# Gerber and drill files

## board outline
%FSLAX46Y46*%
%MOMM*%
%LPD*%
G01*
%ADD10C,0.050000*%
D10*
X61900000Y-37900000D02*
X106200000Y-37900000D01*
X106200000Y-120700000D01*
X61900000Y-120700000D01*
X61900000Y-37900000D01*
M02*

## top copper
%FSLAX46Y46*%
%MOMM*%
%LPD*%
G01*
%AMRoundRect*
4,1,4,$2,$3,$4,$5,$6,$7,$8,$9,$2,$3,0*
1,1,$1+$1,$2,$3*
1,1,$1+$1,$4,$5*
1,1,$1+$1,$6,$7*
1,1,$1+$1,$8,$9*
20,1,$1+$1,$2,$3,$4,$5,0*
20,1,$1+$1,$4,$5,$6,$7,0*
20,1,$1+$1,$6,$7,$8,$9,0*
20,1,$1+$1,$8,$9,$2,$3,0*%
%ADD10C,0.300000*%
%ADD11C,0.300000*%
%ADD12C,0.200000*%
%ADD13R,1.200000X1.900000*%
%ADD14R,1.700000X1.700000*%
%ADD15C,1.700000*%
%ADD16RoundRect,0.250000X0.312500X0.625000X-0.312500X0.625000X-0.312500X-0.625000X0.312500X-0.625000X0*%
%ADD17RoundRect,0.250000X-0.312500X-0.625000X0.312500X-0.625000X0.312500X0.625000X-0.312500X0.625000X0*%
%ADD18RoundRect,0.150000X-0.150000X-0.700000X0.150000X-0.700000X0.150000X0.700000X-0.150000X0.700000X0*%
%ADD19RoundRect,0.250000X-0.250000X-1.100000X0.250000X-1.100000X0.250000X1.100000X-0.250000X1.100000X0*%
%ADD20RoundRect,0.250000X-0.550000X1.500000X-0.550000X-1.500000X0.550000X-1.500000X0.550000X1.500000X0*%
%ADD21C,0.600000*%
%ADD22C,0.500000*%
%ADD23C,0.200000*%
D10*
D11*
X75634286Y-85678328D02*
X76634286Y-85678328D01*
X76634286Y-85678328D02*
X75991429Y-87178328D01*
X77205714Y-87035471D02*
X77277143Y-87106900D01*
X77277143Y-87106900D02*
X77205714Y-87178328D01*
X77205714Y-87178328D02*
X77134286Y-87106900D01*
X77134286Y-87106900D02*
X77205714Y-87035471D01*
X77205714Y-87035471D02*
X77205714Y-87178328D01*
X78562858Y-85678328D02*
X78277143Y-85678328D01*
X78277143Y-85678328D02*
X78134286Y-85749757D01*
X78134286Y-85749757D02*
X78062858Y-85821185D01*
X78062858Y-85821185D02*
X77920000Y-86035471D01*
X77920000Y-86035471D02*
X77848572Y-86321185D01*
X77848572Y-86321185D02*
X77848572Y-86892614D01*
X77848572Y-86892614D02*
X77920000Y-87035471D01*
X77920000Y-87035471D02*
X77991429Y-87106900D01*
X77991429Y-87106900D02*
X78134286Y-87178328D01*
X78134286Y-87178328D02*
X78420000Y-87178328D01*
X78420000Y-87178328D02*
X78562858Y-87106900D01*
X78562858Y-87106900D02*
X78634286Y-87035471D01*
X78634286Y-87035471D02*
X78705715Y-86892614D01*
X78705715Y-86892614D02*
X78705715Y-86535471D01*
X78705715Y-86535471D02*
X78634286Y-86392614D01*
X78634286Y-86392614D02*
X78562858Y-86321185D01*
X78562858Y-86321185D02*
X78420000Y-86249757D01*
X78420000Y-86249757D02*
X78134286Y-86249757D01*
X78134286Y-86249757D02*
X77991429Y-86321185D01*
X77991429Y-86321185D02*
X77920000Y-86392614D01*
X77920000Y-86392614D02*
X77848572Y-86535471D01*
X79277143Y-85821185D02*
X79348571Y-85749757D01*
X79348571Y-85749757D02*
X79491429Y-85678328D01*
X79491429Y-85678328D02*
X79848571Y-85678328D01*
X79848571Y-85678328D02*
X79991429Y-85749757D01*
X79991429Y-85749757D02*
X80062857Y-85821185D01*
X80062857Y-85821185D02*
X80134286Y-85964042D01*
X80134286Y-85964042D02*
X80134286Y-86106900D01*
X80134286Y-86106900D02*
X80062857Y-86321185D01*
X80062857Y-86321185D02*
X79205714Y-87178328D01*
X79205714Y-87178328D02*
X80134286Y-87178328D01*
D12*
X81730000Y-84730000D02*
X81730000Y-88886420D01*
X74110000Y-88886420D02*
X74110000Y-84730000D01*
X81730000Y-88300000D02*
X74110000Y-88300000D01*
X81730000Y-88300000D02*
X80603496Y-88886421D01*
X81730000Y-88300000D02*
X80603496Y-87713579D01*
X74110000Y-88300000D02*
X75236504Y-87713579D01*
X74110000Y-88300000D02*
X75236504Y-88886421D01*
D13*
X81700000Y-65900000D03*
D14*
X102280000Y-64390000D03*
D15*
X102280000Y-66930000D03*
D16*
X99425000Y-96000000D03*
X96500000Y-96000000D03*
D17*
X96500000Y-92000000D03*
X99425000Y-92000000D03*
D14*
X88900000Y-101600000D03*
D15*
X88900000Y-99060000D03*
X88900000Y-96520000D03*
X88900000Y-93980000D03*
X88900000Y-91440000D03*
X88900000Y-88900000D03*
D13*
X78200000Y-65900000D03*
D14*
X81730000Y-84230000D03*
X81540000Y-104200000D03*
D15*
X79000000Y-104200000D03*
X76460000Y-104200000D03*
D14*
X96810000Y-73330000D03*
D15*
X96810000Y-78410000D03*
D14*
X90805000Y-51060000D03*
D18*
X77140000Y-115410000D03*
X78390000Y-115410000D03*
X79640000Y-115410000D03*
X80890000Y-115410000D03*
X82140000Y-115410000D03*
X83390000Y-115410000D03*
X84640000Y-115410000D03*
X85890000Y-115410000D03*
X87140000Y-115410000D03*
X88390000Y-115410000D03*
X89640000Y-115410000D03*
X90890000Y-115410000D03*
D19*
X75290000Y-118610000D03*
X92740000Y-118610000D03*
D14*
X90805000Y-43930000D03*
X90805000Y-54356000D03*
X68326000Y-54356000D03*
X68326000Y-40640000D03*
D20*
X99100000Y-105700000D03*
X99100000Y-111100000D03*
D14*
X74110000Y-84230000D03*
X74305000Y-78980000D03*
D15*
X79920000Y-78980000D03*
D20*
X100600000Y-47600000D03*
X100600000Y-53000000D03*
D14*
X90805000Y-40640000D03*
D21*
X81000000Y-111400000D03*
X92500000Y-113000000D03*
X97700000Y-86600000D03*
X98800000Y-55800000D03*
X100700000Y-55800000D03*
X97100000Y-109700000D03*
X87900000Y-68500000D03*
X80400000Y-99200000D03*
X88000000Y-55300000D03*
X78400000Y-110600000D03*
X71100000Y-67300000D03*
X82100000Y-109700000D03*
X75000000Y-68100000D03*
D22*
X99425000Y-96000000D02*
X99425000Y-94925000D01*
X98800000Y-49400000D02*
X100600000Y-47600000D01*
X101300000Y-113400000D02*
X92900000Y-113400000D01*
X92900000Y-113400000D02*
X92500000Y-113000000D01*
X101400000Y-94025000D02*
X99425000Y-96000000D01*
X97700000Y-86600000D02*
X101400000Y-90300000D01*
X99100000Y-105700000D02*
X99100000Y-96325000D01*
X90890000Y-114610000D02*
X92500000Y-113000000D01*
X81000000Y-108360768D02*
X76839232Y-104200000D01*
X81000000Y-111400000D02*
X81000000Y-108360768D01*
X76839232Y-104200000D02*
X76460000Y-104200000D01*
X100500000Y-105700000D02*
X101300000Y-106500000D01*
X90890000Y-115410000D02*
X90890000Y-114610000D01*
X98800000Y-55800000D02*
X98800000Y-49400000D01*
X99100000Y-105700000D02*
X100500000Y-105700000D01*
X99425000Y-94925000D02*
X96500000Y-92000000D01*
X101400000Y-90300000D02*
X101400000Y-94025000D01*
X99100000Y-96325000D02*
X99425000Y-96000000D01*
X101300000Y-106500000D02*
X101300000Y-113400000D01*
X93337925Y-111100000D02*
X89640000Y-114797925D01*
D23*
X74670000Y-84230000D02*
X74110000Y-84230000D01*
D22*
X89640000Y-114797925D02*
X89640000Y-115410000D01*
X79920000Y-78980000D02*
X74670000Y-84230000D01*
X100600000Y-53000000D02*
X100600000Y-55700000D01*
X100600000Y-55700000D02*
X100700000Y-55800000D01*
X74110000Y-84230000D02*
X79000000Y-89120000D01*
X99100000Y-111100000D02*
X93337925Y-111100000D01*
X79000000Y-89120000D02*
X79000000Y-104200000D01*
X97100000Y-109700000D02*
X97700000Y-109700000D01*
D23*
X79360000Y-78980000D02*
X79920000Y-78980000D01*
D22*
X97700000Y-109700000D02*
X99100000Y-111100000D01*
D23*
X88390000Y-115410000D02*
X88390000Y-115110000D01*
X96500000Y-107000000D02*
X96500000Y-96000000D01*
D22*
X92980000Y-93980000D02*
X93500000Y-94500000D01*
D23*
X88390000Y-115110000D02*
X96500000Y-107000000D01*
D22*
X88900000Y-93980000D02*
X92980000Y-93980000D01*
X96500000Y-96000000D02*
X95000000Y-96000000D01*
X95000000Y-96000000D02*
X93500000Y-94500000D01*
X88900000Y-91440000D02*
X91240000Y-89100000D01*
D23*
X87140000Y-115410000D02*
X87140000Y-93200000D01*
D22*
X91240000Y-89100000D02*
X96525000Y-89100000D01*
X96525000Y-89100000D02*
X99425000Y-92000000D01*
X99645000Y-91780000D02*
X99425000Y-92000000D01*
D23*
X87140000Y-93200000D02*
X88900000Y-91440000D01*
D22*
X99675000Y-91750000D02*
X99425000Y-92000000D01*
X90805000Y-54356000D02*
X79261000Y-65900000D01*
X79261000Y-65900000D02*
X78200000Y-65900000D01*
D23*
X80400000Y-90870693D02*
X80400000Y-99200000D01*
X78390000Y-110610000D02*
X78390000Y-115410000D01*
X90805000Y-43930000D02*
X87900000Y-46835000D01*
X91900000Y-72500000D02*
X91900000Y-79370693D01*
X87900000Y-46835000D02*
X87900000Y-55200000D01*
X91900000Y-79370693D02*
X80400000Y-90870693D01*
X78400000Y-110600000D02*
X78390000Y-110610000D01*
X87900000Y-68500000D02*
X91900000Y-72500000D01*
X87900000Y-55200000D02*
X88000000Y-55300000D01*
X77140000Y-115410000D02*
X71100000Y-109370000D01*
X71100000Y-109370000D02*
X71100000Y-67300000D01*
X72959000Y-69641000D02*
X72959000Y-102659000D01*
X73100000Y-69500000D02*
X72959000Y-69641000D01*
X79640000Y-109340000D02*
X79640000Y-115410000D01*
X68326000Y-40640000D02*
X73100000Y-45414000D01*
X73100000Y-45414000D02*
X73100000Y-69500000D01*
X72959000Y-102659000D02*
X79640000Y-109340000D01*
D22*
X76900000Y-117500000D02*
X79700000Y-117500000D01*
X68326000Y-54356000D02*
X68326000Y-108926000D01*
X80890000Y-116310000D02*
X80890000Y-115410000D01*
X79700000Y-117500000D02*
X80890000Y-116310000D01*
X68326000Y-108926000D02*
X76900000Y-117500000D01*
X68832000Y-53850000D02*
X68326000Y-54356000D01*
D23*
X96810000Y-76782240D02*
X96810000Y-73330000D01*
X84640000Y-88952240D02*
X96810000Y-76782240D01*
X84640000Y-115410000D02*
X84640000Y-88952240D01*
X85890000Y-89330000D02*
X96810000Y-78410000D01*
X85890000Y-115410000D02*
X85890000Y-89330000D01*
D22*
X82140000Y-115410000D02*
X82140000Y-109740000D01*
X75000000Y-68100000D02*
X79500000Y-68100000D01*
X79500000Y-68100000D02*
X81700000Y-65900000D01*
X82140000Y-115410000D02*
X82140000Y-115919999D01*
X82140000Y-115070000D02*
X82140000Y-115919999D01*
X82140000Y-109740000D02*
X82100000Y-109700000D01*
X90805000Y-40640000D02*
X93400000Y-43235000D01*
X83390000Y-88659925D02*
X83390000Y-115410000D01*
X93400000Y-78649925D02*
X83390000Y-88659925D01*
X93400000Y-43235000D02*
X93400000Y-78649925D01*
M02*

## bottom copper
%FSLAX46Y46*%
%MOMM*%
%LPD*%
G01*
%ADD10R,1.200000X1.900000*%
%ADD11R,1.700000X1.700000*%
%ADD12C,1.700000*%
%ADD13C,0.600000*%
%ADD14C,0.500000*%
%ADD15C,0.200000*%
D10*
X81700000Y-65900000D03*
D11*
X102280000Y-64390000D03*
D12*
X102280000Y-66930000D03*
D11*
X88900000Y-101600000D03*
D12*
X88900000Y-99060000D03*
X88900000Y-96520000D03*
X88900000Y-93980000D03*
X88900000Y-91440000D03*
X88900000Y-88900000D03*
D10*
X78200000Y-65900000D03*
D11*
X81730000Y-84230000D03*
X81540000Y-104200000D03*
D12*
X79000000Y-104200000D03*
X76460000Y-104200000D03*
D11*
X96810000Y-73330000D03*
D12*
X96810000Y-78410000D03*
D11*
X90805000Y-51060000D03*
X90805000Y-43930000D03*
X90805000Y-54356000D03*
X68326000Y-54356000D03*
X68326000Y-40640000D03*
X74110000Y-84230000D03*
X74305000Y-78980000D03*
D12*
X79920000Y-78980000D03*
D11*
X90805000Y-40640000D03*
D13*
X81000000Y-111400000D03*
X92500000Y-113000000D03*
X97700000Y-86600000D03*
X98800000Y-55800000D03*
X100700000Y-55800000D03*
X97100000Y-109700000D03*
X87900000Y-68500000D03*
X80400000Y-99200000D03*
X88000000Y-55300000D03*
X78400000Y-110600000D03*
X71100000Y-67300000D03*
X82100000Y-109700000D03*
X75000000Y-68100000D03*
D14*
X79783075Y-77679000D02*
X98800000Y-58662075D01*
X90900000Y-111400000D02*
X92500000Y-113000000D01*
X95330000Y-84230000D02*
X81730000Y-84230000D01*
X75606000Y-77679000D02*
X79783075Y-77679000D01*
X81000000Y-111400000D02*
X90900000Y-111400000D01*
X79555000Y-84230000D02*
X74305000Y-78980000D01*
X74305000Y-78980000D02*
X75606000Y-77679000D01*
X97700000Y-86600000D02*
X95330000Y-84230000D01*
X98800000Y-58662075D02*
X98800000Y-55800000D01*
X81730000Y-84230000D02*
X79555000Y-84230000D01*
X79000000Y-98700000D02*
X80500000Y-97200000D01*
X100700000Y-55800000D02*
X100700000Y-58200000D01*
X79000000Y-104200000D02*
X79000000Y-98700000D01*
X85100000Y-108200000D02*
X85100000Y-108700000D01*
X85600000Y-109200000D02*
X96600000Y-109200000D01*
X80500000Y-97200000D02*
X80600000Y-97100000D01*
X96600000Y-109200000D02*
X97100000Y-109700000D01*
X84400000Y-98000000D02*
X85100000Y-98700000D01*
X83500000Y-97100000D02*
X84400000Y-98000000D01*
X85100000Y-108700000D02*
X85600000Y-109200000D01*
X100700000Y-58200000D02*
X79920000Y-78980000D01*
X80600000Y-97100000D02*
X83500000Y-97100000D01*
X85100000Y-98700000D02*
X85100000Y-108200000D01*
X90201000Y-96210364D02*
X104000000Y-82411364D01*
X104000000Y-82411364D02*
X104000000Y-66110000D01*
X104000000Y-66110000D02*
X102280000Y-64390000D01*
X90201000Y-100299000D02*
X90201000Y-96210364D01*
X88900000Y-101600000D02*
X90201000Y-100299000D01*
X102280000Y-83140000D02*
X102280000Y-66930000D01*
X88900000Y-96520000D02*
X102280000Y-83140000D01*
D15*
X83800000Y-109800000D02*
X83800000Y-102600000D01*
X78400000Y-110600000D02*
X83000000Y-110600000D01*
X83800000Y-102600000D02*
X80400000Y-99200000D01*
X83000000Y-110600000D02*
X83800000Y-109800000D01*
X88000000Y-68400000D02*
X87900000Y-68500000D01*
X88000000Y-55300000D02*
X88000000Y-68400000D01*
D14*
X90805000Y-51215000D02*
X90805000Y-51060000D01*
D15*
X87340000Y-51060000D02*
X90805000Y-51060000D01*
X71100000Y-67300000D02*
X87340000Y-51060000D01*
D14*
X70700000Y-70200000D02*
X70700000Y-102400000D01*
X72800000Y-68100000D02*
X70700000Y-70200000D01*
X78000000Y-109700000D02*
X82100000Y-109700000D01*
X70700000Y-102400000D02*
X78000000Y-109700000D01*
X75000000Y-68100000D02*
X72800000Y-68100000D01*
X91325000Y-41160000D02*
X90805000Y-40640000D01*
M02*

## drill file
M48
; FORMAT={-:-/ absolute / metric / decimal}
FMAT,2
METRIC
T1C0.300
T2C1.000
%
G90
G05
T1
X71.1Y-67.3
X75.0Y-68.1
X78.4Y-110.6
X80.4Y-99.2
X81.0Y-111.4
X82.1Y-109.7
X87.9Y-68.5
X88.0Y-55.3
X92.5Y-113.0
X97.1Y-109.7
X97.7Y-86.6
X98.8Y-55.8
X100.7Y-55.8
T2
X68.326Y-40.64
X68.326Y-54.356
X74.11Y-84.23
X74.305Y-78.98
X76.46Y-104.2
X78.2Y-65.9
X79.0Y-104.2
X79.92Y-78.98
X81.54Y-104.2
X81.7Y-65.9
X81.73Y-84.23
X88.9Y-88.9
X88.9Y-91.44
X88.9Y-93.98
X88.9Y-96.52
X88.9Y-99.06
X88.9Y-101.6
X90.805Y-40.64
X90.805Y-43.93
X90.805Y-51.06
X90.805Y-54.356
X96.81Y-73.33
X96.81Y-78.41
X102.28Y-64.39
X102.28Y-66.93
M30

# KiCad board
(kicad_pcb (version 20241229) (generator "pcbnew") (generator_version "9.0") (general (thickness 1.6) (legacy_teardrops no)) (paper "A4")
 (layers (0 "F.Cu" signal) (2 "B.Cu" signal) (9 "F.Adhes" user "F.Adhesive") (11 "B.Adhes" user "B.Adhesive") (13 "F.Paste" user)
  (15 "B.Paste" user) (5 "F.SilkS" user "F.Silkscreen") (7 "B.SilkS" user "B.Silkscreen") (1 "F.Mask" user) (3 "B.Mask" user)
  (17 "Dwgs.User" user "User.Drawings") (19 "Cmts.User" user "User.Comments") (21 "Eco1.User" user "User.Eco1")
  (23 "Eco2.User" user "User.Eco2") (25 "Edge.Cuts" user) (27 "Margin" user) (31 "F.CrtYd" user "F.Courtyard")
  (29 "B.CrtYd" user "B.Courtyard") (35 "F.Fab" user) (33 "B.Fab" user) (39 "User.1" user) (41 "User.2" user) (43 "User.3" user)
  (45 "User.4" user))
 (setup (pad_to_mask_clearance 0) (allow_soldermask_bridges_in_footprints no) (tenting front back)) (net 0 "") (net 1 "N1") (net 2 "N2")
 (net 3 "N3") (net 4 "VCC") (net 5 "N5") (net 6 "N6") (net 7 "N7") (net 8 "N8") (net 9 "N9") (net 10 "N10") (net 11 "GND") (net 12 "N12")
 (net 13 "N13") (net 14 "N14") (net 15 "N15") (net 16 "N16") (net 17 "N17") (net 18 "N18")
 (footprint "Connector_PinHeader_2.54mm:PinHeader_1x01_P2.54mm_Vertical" (layer "F.Cu") (at 81.7 65.9 90)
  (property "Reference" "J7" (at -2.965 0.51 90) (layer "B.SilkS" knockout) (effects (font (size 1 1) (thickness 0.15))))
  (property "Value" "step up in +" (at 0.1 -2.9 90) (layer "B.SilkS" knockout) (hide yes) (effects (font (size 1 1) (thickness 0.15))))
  (pad "1" thru_hole rect (at 0 0 90) (size 1.9 1.2) (drill 1) (layers "*.Cu" "*.Mask") (remove_unused_layers no) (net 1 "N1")))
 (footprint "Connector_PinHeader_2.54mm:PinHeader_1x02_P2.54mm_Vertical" (layer "F.Cu") (at 102.28 64.39)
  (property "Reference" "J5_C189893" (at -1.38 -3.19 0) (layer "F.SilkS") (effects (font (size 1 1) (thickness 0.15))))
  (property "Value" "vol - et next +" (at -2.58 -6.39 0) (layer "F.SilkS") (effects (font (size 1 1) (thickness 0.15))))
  (pad "1" thru_hole rect (at 0 0) (size 1.7 1.7) (drill 1) (layers "*.Cu" "*.Mask") (remove_unused_layers no) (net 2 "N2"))
  (pad "2" thru_hole circle (at 0 2.54) (size 1.7 1.7) (drill 1) (layers "*.Cu" "*.Mask") (remove_unused_layers no) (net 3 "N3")))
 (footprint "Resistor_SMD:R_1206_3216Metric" (layer "F.Cu") (at 97.9625 96 180)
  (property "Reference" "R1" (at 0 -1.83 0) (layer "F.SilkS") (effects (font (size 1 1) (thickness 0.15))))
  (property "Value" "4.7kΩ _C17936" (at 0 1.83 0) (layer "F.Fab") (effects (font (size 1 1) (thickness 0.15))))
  (pad "1" smd roundrect (at -1.4625 0 180) (size 1.125 1.75) (layers "F.Cu" "F.Mask" "F.Paste") (roundrect_rratio 0.222222) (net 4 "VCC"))
  (pad "2" smd roundrect (at 1.4625 0 180) (size 1.125 1.75) (layers "F.Cu" "F.Mask" "F.Paste") (roundrect_rratio 0.222222) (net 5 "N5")))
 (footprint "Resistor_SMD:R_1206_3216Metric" (layer "F.Cu") (at 97.9625 92)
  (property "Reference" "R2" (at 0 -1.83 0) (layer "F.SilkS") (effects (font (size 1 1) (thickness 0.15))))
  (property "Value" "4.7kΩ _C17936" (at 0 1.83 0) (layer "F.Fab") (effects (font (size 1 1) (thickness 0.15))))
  (pad "1" smd roundrect (at -1.4625 0) (size 1.125 1.75) (layers "F.Cu" "F.Mask" "F.Paste") (roundrect_rratio 0.222222) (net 4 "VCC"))
  (pad "2" smd roundrect (at 1.4625 0) (size 1.125 1.75) (layers "F.Cu" "F.Mask" "F.Paste") (roundrect_rratio 0.222222) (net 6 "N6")))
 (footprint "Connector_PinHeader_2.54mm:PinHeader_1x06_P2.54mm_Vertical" (layer "F.Cu") (at 88.9 101.6 180)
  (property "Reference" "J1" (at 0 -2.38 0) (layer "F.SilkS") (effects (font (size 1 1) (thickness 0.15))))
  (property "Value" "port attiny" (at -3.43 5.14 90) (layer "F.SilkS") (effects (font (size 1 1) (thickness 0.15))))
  (pad "1" thru_hole rect (at 0 0 180) (size 1.7 1.7) (drill 1) (layers "*.Cu" "*.Mask") (remove_unused_layers no) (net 2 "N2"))
  (pad "2" thru_hole circle (at 0 2.54 180) (size 1.7 1.7) (drill 1) (layers "*.Cu" "*.Mask") (remove_unused_layers no) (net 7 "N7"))
  (pad "3" thru_hole circle (at 0 5.08 180) (size 1.7 1.7) (drill 1) (layers "*.Cu" "*.Mask") (remove_unused_layers no) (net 3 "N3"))
  (pad "4" thru_hole circle (at 0 7.62 180) (size 1.7 1.7) (drill 1) (layers "*.Cu" "*.Mask") (remove_unused_layers no) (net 5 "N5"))
  (pad "5" thru_hole circle (at 0 10.16 180) (size 1.7 1.7) (drill 1) (layers "*.Cu" "*.Mask") (remove_unused_layers no) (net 6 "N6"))
  (pad "6" thru_hole circle (at 0 12.7 180) (size 1.7 1.7) (drill 1) (layers "*.Cu" "*.Mask") (remove_unused_layers no) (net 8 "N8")))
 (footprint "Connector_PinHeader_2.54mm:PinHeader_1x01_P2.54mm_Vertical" (layer "F.Cu") (at 78.1 65.9 90)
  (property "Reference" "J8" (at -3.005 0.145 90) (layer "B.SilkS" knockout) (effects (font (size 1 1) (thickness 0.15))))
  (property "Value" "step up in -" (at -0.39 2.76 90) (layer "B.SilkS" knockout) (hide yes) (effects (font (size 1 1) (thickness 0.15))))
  (pad "1" thru_hole rect (at 0 0.1 90) (size 1.9 1.2) (drill 1) (layers "*.Cu" "*.Mask") (remove_unused_layers no) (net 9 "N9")))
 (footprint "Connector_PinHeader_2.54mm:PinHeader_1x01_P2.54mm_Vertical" (layer "F.Cu") (at 81.73 84.23)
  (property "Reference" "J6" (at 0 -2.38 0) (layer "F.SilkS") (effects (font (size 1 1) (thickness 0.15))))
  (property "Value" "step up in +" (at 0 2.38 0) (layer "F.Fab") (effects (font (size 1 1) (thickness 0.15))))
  (pad "1" thru_hole rect (at 0 0) (size 1.7 1.7) (drill 1) (layers "*.Cu" "*.Mask") (remove_unused_layers no) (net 4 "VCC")
   (padstack (mode custom) (layer "B.Cu" (shape rect) (size 1.7 1.7) (zone_connect -1)))))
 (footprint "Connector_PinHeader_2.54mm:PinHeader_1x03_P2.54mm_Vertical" (layer "F.Cu") (at 81.54 104.2 -90)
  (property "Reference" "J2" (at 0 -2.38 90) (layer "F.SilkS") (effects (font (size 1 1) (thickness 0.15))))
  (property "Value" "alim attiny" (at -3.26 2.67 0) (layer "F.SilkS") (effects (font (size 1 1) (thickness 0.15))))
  (pad "1" thru_hole rect (at 0 0 270) (size 1.7 1.7) (drill 1) (layers "*.Cu" "*.Mask") (remove_unused_layers no) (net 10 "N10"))
  (pad "2" thru_hole circle (at 0 2.54 270) (size 1.7 1.7) (drill 1) (layers "*.Cu" "*.Mask") (remove_unused_layers no) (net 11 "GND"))
  (pad "3" thru_hole circle (at 0 5.08 270) (size 1.7 1.7) (drill 1) (layers "*.Cu" "*.Mask") (remove_unused_layers no) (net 4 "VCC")))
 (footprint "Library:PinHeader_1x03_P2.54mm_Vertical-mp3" (layer "F.Cu") (at 96.81 73.33)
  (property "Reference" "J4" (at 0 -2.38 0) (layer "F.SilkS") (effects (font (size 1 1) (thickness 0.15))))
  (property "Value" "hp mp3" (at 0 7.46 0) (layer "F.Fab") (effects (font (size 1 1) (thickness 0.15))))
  (pad "1" thru_hole rect (at 0 0) (size 1.7 1.7) (drill 1) (layers "*.Cu" "*.Mask") (remove_unused_layers no) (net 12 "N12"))
  (pad "2" thru_hole circle (at 0 5.08) (size 1.7 1.7) (drill 1) (layers "*.Cu" "*.Mask") (remove_unused_layers no) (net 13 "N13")))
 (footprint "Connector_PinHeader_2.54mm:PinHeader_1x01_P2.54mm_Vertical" (layer "F.Cu") (at 90.805 51.06)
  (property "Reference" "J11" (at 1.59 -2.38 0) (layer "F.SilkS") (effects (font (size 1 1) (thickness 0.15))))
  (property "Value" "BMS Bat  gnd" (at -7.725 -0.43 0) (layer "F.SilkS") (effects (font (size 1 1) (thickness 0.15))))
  (pad "1" thru_hole rect (at 0 0) (size 1.7 1.7) (drill 1) (layers "*.Cu" "*.Mask") (remove_unused_layers no) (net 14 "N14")))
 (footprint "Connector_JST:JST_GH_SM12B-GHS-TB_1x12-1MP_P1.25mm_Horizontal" (layer "F.Cu") (at 84.015 117.26)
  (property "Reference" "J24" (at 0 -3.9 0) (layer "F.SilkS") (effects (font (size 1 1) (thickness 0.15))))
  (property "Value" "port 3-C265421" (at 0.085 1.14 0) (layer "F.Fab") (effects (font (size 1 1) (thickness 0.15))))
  (pad "1" smd roundrect (at -6.875 -1.85) (size 0.6 1.7) (layers "F.Cu" "F.Mask" "F.Paste") (roundrect_rratio 0.25) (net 14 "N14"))
  (pad "2" smd roundrect (at -5.625 -1.85) (size 0.6 1.7) (layers "F.Cu" "F.Mask" "F.Paste") (roundrect_rratio 0.25) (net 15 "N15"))
  (pad "3" smd roundrect (at -4.375 -1.85) (size 0.6 1.7) (layers "F.Cu" "F.Mask" "F.Paste") (roundrect_rratio 0.25) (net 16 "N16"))
  (pad "4" smd roundrect (at -3.125 -1.85) (size 0.6 1.7) (layers "F.Cu" "F.Mask" "F.Paste") (roundrect_rratio 0.25) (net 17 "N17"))
  (pad "5" smd roundrect (at -1.875 -1.85) (size 0.6 1.7) (layers "F.Cu" "F.Mask" "F.Paste") (roundrect_rratio 0.25) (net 1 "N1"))
  (pad "6" smd roundrect (at -0.625 -1.85) (size 0.6 1.7) (layers "F.Cu" "F.Mask" "F.Paste") (roundrect_rratio 0.25) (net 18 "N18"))
  (pad "7" smd roundrect (at 0.625 -1.85) (size 0.6 1.7) (layers "F.Cu" "F.Mask" "F.Paste") (roundrect_rratio 0.25) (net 12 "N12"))
  (pad "8" smd roundrect (at 1.875 -1.85) (size 0.6 1.7) (layers "F.Cu" "F.Mask" "F.Paste") (roundrect_rratio 0.25) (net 13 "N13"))
  (pad "9" smd roundrect (at 3.125 -1.85) (size 0.6 1.7) (layers "F.Cu" "F.Mask" "F.Paste") (roundrect_rratio 0.25) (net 6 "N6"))
  (pad "10" smd roundrect (at 4.375 -1.85) (size 0.6 1.7) (layers "F.Cu" "F.Mask" "F.Paste") (roundrect_rratio 0.25) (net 5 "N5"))
  (pad "11" smd roundrect (at 5.625 -1.85) (size 0.6 1.7) (layers "F.Cu" "F.Mask" "F.Paste") (roundrect_rratio 0.25) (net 11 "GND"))
  (pad "12" smd roundrect (at 6.875 -1.85) (size 0.6 1.7) (layers "F.Cu" "F.Mask" "F.Paste") (roundrect_rratio 0.25) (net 4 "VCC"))
  (pad "MP" smd roundrect (at -8.725 1.35) (size 1 2.7) (layers "F.Cu" "F.Mask" "F.Paste") (roundrect_rratio 0.25))
  (pad "MP" smd roundrect (at 8.725 1.35) (size 1 2.7) (layers "F.Cu" "F.Mask" "F.Paste") (roundrect_rratio 0.25)))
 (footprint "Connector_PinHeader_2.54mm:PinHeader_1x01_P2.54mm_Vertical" (layer "F.Cu") (at 90.805 43.93)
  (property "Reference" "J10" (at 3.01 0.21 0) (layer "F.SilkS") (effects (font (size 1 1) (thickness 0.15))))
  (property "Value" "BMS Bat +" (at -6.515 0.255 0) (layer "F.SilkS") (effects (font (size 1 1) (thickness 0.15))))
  (pad "1" thru_hole rect (at 0 0) (size 1.7 1.7) (drill 1) (layers "*.Cu" "*.Mask") (remove_unused_layers no) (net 15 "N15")))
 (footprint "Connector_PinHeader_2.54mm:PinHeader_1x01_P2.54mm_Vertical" (layer "F.Cu") (at 90.805 54.356)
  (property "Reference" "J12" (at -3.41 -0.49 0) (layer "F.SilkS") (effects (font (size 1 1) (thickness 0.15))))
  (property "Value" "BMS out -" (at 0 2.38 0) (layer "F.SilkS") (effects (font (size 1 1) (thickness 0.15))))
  (pad "1" thru_hole rect (at 0 0) (size 1.7 1.7) (drill 1) (layers "*.Cu" "*.Mask") (remove_unused_layers no) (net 9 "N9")))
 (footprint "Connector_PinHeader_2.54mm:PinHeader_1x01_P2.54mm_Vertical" (layer "F.Cu") (at 68.326 54.356)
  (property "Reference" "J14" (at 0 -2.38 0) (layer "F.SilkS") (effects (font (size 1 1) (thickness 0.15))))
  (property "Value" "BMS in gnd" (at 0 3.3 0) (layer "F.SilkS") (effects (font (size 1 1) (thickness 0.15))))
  (pad "1" thru_hole rect (at 0 0) (size 1.7 1.7) (drill 1) (layers "*.Cu" "*.Mask") (remove_unused_layers no) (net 17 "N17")))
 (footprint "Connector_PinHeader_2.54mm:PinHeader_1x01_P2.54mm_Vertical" (layer "F.Cu") (at 68.326 40.64)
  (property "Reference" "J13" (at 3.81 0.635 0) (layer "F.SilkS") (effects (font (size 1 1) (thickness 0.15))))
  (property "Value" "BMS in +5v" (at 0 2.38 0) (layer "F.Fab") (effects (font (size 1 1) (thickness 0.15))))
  (pad "1" thru_hole rect (at 0 0) (size 1.7 1.7) (drill 1) (layers "*.Cu" "*.Mask") (remove_unused_layers no) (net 16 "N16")))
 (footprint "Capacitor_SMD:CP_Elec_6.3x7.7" (layer "F.Cu") (at 99.1 108.4 -90)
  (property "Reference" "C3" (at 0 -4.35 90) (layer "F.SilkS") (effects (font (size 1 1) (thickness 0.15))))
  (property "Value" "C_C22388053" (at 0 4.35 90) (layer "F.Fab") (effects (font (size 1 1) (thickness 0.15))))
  (pad "1" smd roundrect (at -2.7 0 270) (size 3.5 1.6) (layers "F.Cu" "F.Mask" "F.Paste") (roundrect_rratio 0.15625) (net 4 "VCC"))
  (pad "2" smd roundrect (at 2.7 0 270) (size 3.5 1.6) (layers "F.Cu" "F.Mask" "F.Paste") (roundrect_rratio 0.15625) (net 11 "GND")))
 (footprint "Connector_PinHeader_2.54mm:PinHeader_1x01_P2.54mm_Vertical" (layer "F.Cu") (at 74.11 84.23)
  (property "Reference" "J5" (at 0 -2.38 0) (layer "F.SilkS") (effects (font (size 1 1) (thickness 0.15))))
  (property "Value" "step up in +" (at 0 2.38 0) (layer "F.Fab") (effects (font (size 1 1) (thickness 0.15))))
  (pad "1" thru_hole rect (at 0 0) (size 1.7 1.7) (drill 1) (layers "*.Cu" "*.Mask") (remove_unused_layers no) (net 11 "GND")))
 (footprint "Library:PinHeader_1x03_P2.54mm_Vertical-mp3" (layer "F.Cu") (at 74.84 78.98 90)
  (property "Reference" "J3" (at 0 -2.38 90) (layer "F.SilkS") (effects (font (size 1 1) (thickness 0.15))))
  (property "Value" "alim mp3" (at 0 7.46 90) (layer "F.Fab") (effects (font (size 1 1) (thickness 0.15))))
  (pad "1" thru_hole rect (at 0 -0.535 90) (size 1.7 1.7) (drill 1) (layers "*.Cu" "*.Mask") (remove_unused_layers no) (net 4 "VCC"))
  (pad "2" thru_hole circle (at 0 5.08 90) (size 1.7 1.7) (drill 1) (layers "*.Cu" "*.Mask") (remove_unused_layers no) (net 11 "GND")))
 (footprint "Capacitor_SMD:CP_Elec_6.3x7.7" (layer "F.Cu") (at 100.6 50.3 -90)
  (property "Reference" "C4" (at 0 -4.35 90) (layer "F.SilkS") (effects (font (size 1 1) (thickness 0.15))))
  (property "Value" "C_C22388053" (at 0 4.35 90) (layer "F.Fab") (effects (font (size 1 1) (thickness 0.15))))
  (pad "1" smd roundrect (at -2.7 0 270) (size 3.5 1.6) (layers "F.Cu" "F.Mask" "F.Paste") (roundrect_rratio 0.15625) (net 4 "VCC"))
  (pad "2" smd roundrect (at 2.7 0 270) (size 3.5 1.6) (layers "F.Cu" "F.Mask" "F.Paste") (roundrect_rratio 0.15625) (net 11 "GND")))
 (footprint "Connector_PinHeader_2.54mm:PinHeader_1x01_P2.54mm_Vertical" (layer "F.Cu") (at 90.805 40.64)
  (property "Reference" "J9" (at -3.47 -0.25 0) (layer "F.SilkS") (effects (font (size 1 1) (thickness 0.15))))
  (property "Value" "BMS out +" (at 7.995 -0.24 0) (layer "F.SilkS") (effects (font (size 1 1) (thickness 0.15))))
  (pad "1" thru_hole rect (at 0 0) (size 1.7 1.7) (drill 1) (layers "*.Cu" "*.Mask") (remove_unused_layers no) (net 18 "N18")))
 (gr_rect (start 61.9 37.9) (end 106.2 120.7) (stroke (width 0.05) (type solid)) (fill no) (layer "Edge.Cuts"))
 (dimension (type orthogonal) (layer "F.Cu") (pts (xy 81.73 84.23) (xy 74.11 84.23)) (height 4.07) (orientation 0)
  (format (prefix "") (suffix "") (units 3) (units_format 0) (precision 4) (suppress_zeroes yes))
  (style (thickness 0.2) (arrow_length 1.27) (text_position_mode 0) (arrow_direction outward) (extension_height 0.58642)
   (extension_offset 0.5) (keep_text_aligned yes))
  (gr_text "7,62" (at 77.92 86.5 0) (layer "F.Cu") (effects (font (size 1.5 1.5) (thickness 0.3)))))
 (segment (start 99.425 96) (end 99.425 94.925) (width 0.5) (layer "F.Cu") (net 4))
 (segment (start 98.8 49.4) (end 100.6 47.6) (width 0.5) (layer "F.Cu") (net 4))
 (segment (start 101.3 113.4) (end 92.9 113.4) (width 0.5) (layer "F.Cu") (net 4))
 (segment (start 92.9 113.4) (end 92.5 113) (width 0.5) (layer "F.Cu") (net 4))
 (segment (start 101.4 94.025) (end 99.425 96) (width 0.5) (layer "F.Cu") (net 4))
 (segment (start 97.7 86.6) (end 101.4 90.3) (width 0.5) (layer "F.Cu") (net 4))
 (segment (start 99.1 105.7) (end 99.1 96.325) (width 0.5) (layer "F.Cu") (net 4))
 (segment (start 90.89 114.61) (end 92.5 113) (width 0.5) (layer "F.Cu") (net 4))
 (segment (start 81 108.360768) (end 76.839232 104.2) (width 0.5) (layer "F.Cu") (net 4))
 (segment (start 81 111.4) (end 81 108.360768) (width 0.5) (layer "F.Cu") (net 4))
 (segment (start 76.839232 104.2) (end 76.46 104.2) (width 0.5) (layer "F.Cu") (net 4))
 (segment (start 100.5 105.7) (end 101.3 106.5) (width 0.5) (layer "F.Cu") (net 4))
 (segment (start 90.89 115.41) (end 90.89 114.61) (width 0.5) (layer "F.Cu") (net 4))
 (segment (start 98.8 55.8) (end 98.8 49.4) (width 0.5) (layer "F.Cu") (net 4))
 (segment (start 99.1 105.7) (end 100.5 105.7) (width 0.5) (layer "F.Cu") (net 4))
 (segment (start 99.425 94.925) (end 96.5 92) (width 0.5) (layer "F.Cu") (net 4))
 (segment (start 101.4 90.3) (end 101.4 94.025) (width 0.5) (layer "F.Cu") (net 4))
 (segment (start 99.1 96.325) (end 99.425 96) (width 0.5) (layer "F.Cu") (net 4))
 (segment (start 101.3 106.5) (end 101.3 113.4) (width 0.5) (layer "F.Cu") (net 4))
 (via (at 81 111.4) (size 0.6) (drill 0.3) (layers "F.Cu" "B.Cu") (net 4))
 (via (at 92.5 113) (size 0.6) (drill 0.3) (layers "F.Cu" "B.Cu") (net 4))
 (via (at 97.7 86.6) (size 0.6) (drill 0.3) (layers "F.Cu" "B.Cu") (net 4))
 (via (at 98.8 55.8) (size 0.6) (drill 0.3) (layers "F.Cu" "B.Cu") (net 4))
 (segment (start 79.783075 77.679) (end 98.8 58.662075) (width 0.5) (layer "B.Cu") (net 4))
 (segment (start 90.9 111.4) (end 92.5 113) (width 0.5) (layer "B.Cu") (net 4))
 (segment (start 95.33 84.23) (end 81.73 84.23) (width 0.5) (layer "B.Cu") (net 4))
 (segment (start 75.606 77.679) (end 79.783075 77.679) (width 0.5) (layer "B.Cu") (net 4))
 (segment (start 81 111.4) (end 90.9 111.4) (width 0.5) (layer "B.Cu") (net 4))
 (segment (start 79.555 84.23) (end 74.305 78.98) (width 0.5) (layer "B.Cu") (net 4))
 (segment (start 74.305 78.98) (end 75.606 77.679) (width 0.5) (layer "B.Cu") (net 4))
 (segment (start 97.7 86.6) (end 95.33 84.23) (width 0.5) (layer "B.Cu") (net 4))
 (segment (start 98.8 58.662075) (end 98.8 55.8) (width 0.5) (layer "B.Cu") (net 4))
 (segment (start 81.73 84.23) (end 79.555 84.23) (width 0.5) (layer "B.Cu") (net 4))
 (segment (start 93.337925 111.1) (end 89.64 114.797925) (width 0.5) (layer "F.Cu") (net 11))
 (segment (start 74.67 84.23) (end 74.11 84.23) (width 0.2) (layer "F.Cu") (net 11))
 (segment (start 89.64 114.797925) (end 89.64 115.41) (width 0.5) (layer "F.Cu") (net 11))
 (segment (start 79.92 78.98) (end 74.67 84.23) (width 0.5) (layer "F.Cu") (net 11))
 (segment (start 100.6 53) (end 100.6 55.7) (width 0.5) (layer "F.Cu") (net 11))
 (segment (start 100.6 55.7) (end 100.7 55.8) (width 0.5) (layer "F.Cu") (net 11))
 (segment (start 74.11 84.23) (end 79 89.12) (width 0.5) (layer "F.Cu") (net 11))
 (segment (start 99.1 111.1) (end 93.337925 111.1) (width 0.5) (layer "F.Cu") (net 11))
 (segment (start 79 89.12) (end 79 104.2) (width 0.5) (layer "F.Cu") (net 11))
 (segment (start 97.1 109.7) (end 97.7 109.7) (width 0.5) (layer "F.Cu") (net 11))
 (segment (start 79.36 78.98) (end 79.92 78.98) (width 0.2) (layer "F.Cu") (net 11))
 (segment (start 97.7 109.7) (end 99.1 111.1) (width 0.5) (layer "F.Cu") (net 11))
 (via (at 100.7 55.8) (size 0.6) (drill 0.3) (layers "F.Cu" "B.Cu") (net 11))
 (via (at 97.1 109.7) (size 0.6) (drill 0.3) (layers "F.Cu" "B.Cu") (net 11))
 (segment (start 79 98.7) (end 80.5 97.2) (width 0.5) (layer "B.Cu") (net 11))
 (segment (start 100.7 55.8) (end 100.7 58.2) (width 0.5) (layer "B.Cu") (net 11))
 (segment (start 79 104.2) (end 79 98.7) (width 0.5) (layer "B.Cu") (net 11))
 (segment (start 85.1 108.2) (end 85.1 108.7) (width 0.5) (layer "B.Cu") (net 11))
 (segment (start 85.6 109.2) (end 96.6 109.2) (width 0.5) (layer "B.Cu") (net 11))
 (segment (start 80.5 97.2) (end 80.6 97.1) (width 0.5) (layer "B.Cu") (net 11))
 (segment (start 96.6 109.2) (end 97.1 109.7) (width 0.5) (layer "B.Cu") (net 11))
 (segment (start 84.4 98) (end 85.1 98.7) (width 0.5) (layer "B.Cu") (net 11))
 (segment (start 83.5 97.1) (end 84.4 98) (width 0.5) (layer "B.Cu") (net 11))
 (segment (start 85.1 108.7) (end 85.6 109.2) (width 0.5) (layer "B.Cu") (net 11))
 (segment (start 100.7 58.2) (end 79.92 78.98) (width 0.5) (layer "B.Cu") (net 11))
 (segment (start 80.6 97.1) (end 83.5 97.1) (width 0.5) (layer "B.Cu") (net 11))
 (segment (start 85.1 98.7) (end 85.1 108.2) (width 0.5) (layer "B.Cu") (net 11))
 (segment (start 88.39 115.41) (end 88.39 115.11) (width 0.2) (layer "F.Cu") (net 5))
 (segment (start 96.5 107) (end 96.5 96) (width 0.2) (layer "F.Cu") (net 5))
 (segment (start 92.98 93.98) (end 93.5 94.5) (width 0.5) (layer "F.Cu") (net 5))
 (segment (start 88.39 115.11) (end 96.5 107) (width 0.2) (layer "F.Cu") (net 5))
 (segment (start 88.9 93.98) (end 92.98 93.98) (width 0.5) (layer "F.Cu") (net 5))
 (segment (start 96.5 96) (end 95 96) (width 0.5) (layer "F.Cu") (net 5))
 (segment (start 95 96) (end 93.5 94.5) (width 0.5) (layer "F.Cu") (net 5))
 (segment (start 88.9 91.44) (end 91.24 89.1) (width 0.5) (layer "F.Cu") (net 6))
 (segment (start 87.14 115.41) (end 87.14 93.2) (width 0.2) (layer "F.Cu") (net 6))
 (segment (start 91.24 89.1) (end 96.525 89.1) (width 0.5) (layer "F.Cu") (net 6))
 (segment (start 96.525 89.1) (end 99.425 92) (width 0.5) (layer "F.Cu") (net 6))
 (segment (start 99.645 91.78) (end 99.425 92) (width 0.5) (layer "F.Cu") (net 6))
 (segment (start 87.14 93.2) (end 88.9 91.44) (width 0.2) (layer "F.Cu") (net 6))
 (segment (start 99.675 91.75) (end 99.425 92) (width 0.5) (layer "F.Cu") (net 6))
 (segment (start 90.201 96.210364) (end 104 82.411364) (width 0.5) (layer "B.Cu") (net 2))
 (segment (start 104 82.411364) (end 104 66.11) (width 0.5) (layer "B.Cu") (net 2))
 (segment (start 104 66.11) (end 102.28 64.39) (width 0.5) (layer "B.Cu") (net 2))
 (segment (start 90.201 100.299) (end 90.201 96.210364) (width 0.5) (layer "B.Cu") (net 2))
 (segment (start 88.9 101.6) (end 90.201 100.299) (width 0.5) (layer "B.Cu") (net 2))
 (segment (start 102.28 83.14) (end 102.28 66.93) (width 0.5) (layer "B.Cu") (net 3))
 (segment (start 88.9 96.52) (end 102.28 83.14) (width 0.5) (layer "B.Cu") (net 3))
 (segment (start 90.805 54.356) (end 79.261 65.9) (width 0.5) (layer "F.Cu") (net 9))
 (segment (start 79.261 65.9) (end 78.2 65.9) (width 0.5) (layer "F.Cu") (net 9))
 (segment (start 80.4 90.870693) (end 80.4 99.2) (width 0.2) (layer "F.Cu") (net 15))
 (segment (start 78.39 110.61) (end 78.39 115.41) (width 0.2) (layer "F.Cu") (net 15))
 (segment (start 90.805 43.93) (end 87.9 46.835) (width 0.2) (layer "F.Cu") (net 15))
 (segment (start 91.9 72.5) (end 91.9 79.370693) (width 0.2) (layer "F.Cu") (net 15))
 (segment (start 87.9 46.835) (end 87.9 55.2) (width 0.2) (layer "F.Cu") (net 15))
 (segment (start 91.9 79.370693) (end 80.4 90.870693) (width 0.2) (layer "F.Cu") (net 15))
 (segment (start 78.4 110.6) (end 78.39 110.61) (width 0.2) (layer "F.Cu") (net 15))
 (segment (start 87.9 68.5) (end 91.9 72.5) (width 0.2) (layer "F.Cu") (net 15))
 (segment (start 87.9 55.2) (end 88 55.3) (width 0.2) (layer "F.Cu") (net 15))
 (via (at 87.9 68.5) (size 0.6) (drill 0.3) (layers "F.Cu" "B.Cu") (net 15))
 (via (at 80.4 99.2) (size 0.6) (drill 0.3) (layers "F.Cu" "B.Cu") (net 15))
 (via (at 88 55.3) (size 0.6) (drill 0.3) (layers "F.Cu" "B.Cu") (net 15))
 (via (at 78.4 110.6) (size 0.6) (drill 0.3) (layers "F.Cu" "B.Cu") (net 15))
 (segment (start 83.8 109.8) (end 83.8 102.6) (width 0.2) (layer "B.Cu") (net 15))
 (segment (start 78.4 110.6) (end 83 110.6) (width 0.2) (layer "B.Cu") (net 15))
 (segment (start 83.8 102.6) (end 80.4 99.2) (width 0.2) (layer "B.Cu") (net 15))
 (segment (start 83 110.6) (end 83.8 109.8) (width 0.2) (layer "B.Cu") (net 15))
 (segment (start 88 68.4) (end 87.9 68.5) (width 0.2) (layer "B.Cu") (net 15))
 (segment (start 88 55.3) (end 88 68.4) (width 0.2) (layer "B.Cu") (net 15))
 (segment (start 77.14 115.41) (end 71.1 109.37) (width 0.2) (layer "F.Cu") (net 14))
 (segment (start 71.1 109.37) (end 71.1 67.3) (width 0.2) (layer "F.Cu") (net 14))
 (via (at 71.1 67.3) (size 0.6) (drill 0.3) (layers "F.Cu" "B.Cu") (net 14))
 (segment (start 90.805 51.215) (end 90.805 51.06) (width 0.5) (layer "B.Cu") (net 14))
 (segment (start 87.34 51.06) (end 90.805 51.06) (width 0.2) (layer "B.Cu") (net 14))
 (segment (start 71.1 67.3) (end 87.34 51.06) (width 0.2) (layer "B.Cu") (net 14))
 (segment (start 72.959 69.641) (end 72.959 102.659) (width 0.2) (layer "F.Cu") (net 16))
 (segment (start 73.1 69.5) (end 72.959 69.641) (width 0.2) (layer "F.Cu") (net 16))
 (segment (start 79.64 109.34) (end 79.64 115.41) (width 0.2) (layer "F.Cu") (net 16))
 (segment (start 68.326 40.64) (end 73.1 45.414) (width 0.2) (layer "F.Cu") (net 16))
 (segment (start 73.1 45.414) (end 73.1 69.5) (width 0.2) (layer "F.Cu") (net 16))
 (segment (start 72.959 102.659) (end 79.64 109.34) (width 0.2) (layer "F.Cu") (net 16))
 (segment (start 76.9 117.5) (end 79.7 117.5) (width 0.5) (layer "F.Cu") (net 17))
 (segment (start 68.326 54.356) (end 68.326 108.926) (width 0.5) (layer "F.Cu") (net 17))
 (segment (start 80.89 116.31) (end 80.89 115.41) (width 0.5) (layer "F.Cu") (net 17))
 (segment (start 79.7 117.5) (end 80.89 116.31) (width 0.5) (layer "F.Cu") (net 17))
 (segment (start 68.326 108.926) (end 76.9 117.5) (width 0.5) (layer "F.Cu") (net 17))
 (segment (start 68.832 53.85) (end 68.326 54.356) (width 0.5) (layer "F.Cu") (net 17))
 (segment (start 96.81 76.78224) (end 96.81 73.33) (width 0.2) (layer "F.Cu") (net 12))
 (segment (start 84.64 88.95224) (end 96.81 76.78224) (width 0.2) (layer "F.Cu") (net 12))
 (segment (start 84.64 115.41) (end 84.64 88.95224) (width 0.2) (layer "F.Cu") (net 12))
 (segment (start 85.89 89.33) (end 96.81 78.41) (width 0.2) (layer "F.Cu") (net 13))
 (segment (start 85.89 115.41) (end 85.89 89.33) (width 0.2) (layer "F.Cu") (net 13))
 (segment (start 82.14 115.41) (end 82.14 109.74) (width 0.5) (layer "F.Cu") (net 1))
 (segment (start 75 68.1) (end 79.5 68.1) (width 0.5) (layer "F.Cu") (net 1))
 (segment (start 79.5 68.1) (end 81.7 65.9) (width 0.5) (layer "F.Cu") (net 1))
 (segment (start 82.14 115.41) (end 82.14 115.919999) (width 0.5) (layer "F.Cu") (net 1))
 (segment (start 82.14 115.07) (end 82.14 115.919999) (width 0.5) (layer "F.Cu") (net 1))
 (segment (start 82.14 109.74) (end 82.1 109.7) (width 0.5) (layer "F.Cu") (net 1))
 (via (at 82.1 109.7) (size 0.6) (drill 0.3) (layers "F.Cu" "B.Cu") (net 1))
 (via (at 75 68.1) (size 0.6) (drill 0.3) (layers "F.Cu" "B.Cu") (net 1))
 (segment (start 70.7 70.2) (end 70.7 102.4) (width 0.5) (layer "B.Cu") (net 1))
 (segment (start 72.8 68.1) (end 70.7 70.2) (width 0.5) (layer "B.Cu") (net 1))
 (segment (start 78 109.7) (end 82.1 109.7) (width 0.5) (layer "B.Cu") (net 1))
 (segment (start 70.7 102.4) (end 78 109.7) (width 0.5) (layer "B.Cu") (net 1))
 (segment (start 75 68.1) (end 72.8 68.1) (width 0.5) (layer "B.Cu") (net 1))
 (segment (start 90.805 40.64) (end 93.4 43.235) (width 0.5) (layer "F.Cu") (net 18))
 (segment (start 83.39 88.659925) (end 83.39 115.41) (width 0.5) (layer "F.Cu") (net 18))
 (segment (start 93.4 78.649925) (end 83.39 88.659925) (width 0.5) (layer "F.Cu") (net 18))
 (segment (start 93.4 43.235) (end 93.4 78.649925) (width 0.5) (layer "F.Cu") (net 18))
 (segment (start 91.325 41.16) (end 90.805 40.64) (width 0.5) (layer "B.Cu") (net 18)))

